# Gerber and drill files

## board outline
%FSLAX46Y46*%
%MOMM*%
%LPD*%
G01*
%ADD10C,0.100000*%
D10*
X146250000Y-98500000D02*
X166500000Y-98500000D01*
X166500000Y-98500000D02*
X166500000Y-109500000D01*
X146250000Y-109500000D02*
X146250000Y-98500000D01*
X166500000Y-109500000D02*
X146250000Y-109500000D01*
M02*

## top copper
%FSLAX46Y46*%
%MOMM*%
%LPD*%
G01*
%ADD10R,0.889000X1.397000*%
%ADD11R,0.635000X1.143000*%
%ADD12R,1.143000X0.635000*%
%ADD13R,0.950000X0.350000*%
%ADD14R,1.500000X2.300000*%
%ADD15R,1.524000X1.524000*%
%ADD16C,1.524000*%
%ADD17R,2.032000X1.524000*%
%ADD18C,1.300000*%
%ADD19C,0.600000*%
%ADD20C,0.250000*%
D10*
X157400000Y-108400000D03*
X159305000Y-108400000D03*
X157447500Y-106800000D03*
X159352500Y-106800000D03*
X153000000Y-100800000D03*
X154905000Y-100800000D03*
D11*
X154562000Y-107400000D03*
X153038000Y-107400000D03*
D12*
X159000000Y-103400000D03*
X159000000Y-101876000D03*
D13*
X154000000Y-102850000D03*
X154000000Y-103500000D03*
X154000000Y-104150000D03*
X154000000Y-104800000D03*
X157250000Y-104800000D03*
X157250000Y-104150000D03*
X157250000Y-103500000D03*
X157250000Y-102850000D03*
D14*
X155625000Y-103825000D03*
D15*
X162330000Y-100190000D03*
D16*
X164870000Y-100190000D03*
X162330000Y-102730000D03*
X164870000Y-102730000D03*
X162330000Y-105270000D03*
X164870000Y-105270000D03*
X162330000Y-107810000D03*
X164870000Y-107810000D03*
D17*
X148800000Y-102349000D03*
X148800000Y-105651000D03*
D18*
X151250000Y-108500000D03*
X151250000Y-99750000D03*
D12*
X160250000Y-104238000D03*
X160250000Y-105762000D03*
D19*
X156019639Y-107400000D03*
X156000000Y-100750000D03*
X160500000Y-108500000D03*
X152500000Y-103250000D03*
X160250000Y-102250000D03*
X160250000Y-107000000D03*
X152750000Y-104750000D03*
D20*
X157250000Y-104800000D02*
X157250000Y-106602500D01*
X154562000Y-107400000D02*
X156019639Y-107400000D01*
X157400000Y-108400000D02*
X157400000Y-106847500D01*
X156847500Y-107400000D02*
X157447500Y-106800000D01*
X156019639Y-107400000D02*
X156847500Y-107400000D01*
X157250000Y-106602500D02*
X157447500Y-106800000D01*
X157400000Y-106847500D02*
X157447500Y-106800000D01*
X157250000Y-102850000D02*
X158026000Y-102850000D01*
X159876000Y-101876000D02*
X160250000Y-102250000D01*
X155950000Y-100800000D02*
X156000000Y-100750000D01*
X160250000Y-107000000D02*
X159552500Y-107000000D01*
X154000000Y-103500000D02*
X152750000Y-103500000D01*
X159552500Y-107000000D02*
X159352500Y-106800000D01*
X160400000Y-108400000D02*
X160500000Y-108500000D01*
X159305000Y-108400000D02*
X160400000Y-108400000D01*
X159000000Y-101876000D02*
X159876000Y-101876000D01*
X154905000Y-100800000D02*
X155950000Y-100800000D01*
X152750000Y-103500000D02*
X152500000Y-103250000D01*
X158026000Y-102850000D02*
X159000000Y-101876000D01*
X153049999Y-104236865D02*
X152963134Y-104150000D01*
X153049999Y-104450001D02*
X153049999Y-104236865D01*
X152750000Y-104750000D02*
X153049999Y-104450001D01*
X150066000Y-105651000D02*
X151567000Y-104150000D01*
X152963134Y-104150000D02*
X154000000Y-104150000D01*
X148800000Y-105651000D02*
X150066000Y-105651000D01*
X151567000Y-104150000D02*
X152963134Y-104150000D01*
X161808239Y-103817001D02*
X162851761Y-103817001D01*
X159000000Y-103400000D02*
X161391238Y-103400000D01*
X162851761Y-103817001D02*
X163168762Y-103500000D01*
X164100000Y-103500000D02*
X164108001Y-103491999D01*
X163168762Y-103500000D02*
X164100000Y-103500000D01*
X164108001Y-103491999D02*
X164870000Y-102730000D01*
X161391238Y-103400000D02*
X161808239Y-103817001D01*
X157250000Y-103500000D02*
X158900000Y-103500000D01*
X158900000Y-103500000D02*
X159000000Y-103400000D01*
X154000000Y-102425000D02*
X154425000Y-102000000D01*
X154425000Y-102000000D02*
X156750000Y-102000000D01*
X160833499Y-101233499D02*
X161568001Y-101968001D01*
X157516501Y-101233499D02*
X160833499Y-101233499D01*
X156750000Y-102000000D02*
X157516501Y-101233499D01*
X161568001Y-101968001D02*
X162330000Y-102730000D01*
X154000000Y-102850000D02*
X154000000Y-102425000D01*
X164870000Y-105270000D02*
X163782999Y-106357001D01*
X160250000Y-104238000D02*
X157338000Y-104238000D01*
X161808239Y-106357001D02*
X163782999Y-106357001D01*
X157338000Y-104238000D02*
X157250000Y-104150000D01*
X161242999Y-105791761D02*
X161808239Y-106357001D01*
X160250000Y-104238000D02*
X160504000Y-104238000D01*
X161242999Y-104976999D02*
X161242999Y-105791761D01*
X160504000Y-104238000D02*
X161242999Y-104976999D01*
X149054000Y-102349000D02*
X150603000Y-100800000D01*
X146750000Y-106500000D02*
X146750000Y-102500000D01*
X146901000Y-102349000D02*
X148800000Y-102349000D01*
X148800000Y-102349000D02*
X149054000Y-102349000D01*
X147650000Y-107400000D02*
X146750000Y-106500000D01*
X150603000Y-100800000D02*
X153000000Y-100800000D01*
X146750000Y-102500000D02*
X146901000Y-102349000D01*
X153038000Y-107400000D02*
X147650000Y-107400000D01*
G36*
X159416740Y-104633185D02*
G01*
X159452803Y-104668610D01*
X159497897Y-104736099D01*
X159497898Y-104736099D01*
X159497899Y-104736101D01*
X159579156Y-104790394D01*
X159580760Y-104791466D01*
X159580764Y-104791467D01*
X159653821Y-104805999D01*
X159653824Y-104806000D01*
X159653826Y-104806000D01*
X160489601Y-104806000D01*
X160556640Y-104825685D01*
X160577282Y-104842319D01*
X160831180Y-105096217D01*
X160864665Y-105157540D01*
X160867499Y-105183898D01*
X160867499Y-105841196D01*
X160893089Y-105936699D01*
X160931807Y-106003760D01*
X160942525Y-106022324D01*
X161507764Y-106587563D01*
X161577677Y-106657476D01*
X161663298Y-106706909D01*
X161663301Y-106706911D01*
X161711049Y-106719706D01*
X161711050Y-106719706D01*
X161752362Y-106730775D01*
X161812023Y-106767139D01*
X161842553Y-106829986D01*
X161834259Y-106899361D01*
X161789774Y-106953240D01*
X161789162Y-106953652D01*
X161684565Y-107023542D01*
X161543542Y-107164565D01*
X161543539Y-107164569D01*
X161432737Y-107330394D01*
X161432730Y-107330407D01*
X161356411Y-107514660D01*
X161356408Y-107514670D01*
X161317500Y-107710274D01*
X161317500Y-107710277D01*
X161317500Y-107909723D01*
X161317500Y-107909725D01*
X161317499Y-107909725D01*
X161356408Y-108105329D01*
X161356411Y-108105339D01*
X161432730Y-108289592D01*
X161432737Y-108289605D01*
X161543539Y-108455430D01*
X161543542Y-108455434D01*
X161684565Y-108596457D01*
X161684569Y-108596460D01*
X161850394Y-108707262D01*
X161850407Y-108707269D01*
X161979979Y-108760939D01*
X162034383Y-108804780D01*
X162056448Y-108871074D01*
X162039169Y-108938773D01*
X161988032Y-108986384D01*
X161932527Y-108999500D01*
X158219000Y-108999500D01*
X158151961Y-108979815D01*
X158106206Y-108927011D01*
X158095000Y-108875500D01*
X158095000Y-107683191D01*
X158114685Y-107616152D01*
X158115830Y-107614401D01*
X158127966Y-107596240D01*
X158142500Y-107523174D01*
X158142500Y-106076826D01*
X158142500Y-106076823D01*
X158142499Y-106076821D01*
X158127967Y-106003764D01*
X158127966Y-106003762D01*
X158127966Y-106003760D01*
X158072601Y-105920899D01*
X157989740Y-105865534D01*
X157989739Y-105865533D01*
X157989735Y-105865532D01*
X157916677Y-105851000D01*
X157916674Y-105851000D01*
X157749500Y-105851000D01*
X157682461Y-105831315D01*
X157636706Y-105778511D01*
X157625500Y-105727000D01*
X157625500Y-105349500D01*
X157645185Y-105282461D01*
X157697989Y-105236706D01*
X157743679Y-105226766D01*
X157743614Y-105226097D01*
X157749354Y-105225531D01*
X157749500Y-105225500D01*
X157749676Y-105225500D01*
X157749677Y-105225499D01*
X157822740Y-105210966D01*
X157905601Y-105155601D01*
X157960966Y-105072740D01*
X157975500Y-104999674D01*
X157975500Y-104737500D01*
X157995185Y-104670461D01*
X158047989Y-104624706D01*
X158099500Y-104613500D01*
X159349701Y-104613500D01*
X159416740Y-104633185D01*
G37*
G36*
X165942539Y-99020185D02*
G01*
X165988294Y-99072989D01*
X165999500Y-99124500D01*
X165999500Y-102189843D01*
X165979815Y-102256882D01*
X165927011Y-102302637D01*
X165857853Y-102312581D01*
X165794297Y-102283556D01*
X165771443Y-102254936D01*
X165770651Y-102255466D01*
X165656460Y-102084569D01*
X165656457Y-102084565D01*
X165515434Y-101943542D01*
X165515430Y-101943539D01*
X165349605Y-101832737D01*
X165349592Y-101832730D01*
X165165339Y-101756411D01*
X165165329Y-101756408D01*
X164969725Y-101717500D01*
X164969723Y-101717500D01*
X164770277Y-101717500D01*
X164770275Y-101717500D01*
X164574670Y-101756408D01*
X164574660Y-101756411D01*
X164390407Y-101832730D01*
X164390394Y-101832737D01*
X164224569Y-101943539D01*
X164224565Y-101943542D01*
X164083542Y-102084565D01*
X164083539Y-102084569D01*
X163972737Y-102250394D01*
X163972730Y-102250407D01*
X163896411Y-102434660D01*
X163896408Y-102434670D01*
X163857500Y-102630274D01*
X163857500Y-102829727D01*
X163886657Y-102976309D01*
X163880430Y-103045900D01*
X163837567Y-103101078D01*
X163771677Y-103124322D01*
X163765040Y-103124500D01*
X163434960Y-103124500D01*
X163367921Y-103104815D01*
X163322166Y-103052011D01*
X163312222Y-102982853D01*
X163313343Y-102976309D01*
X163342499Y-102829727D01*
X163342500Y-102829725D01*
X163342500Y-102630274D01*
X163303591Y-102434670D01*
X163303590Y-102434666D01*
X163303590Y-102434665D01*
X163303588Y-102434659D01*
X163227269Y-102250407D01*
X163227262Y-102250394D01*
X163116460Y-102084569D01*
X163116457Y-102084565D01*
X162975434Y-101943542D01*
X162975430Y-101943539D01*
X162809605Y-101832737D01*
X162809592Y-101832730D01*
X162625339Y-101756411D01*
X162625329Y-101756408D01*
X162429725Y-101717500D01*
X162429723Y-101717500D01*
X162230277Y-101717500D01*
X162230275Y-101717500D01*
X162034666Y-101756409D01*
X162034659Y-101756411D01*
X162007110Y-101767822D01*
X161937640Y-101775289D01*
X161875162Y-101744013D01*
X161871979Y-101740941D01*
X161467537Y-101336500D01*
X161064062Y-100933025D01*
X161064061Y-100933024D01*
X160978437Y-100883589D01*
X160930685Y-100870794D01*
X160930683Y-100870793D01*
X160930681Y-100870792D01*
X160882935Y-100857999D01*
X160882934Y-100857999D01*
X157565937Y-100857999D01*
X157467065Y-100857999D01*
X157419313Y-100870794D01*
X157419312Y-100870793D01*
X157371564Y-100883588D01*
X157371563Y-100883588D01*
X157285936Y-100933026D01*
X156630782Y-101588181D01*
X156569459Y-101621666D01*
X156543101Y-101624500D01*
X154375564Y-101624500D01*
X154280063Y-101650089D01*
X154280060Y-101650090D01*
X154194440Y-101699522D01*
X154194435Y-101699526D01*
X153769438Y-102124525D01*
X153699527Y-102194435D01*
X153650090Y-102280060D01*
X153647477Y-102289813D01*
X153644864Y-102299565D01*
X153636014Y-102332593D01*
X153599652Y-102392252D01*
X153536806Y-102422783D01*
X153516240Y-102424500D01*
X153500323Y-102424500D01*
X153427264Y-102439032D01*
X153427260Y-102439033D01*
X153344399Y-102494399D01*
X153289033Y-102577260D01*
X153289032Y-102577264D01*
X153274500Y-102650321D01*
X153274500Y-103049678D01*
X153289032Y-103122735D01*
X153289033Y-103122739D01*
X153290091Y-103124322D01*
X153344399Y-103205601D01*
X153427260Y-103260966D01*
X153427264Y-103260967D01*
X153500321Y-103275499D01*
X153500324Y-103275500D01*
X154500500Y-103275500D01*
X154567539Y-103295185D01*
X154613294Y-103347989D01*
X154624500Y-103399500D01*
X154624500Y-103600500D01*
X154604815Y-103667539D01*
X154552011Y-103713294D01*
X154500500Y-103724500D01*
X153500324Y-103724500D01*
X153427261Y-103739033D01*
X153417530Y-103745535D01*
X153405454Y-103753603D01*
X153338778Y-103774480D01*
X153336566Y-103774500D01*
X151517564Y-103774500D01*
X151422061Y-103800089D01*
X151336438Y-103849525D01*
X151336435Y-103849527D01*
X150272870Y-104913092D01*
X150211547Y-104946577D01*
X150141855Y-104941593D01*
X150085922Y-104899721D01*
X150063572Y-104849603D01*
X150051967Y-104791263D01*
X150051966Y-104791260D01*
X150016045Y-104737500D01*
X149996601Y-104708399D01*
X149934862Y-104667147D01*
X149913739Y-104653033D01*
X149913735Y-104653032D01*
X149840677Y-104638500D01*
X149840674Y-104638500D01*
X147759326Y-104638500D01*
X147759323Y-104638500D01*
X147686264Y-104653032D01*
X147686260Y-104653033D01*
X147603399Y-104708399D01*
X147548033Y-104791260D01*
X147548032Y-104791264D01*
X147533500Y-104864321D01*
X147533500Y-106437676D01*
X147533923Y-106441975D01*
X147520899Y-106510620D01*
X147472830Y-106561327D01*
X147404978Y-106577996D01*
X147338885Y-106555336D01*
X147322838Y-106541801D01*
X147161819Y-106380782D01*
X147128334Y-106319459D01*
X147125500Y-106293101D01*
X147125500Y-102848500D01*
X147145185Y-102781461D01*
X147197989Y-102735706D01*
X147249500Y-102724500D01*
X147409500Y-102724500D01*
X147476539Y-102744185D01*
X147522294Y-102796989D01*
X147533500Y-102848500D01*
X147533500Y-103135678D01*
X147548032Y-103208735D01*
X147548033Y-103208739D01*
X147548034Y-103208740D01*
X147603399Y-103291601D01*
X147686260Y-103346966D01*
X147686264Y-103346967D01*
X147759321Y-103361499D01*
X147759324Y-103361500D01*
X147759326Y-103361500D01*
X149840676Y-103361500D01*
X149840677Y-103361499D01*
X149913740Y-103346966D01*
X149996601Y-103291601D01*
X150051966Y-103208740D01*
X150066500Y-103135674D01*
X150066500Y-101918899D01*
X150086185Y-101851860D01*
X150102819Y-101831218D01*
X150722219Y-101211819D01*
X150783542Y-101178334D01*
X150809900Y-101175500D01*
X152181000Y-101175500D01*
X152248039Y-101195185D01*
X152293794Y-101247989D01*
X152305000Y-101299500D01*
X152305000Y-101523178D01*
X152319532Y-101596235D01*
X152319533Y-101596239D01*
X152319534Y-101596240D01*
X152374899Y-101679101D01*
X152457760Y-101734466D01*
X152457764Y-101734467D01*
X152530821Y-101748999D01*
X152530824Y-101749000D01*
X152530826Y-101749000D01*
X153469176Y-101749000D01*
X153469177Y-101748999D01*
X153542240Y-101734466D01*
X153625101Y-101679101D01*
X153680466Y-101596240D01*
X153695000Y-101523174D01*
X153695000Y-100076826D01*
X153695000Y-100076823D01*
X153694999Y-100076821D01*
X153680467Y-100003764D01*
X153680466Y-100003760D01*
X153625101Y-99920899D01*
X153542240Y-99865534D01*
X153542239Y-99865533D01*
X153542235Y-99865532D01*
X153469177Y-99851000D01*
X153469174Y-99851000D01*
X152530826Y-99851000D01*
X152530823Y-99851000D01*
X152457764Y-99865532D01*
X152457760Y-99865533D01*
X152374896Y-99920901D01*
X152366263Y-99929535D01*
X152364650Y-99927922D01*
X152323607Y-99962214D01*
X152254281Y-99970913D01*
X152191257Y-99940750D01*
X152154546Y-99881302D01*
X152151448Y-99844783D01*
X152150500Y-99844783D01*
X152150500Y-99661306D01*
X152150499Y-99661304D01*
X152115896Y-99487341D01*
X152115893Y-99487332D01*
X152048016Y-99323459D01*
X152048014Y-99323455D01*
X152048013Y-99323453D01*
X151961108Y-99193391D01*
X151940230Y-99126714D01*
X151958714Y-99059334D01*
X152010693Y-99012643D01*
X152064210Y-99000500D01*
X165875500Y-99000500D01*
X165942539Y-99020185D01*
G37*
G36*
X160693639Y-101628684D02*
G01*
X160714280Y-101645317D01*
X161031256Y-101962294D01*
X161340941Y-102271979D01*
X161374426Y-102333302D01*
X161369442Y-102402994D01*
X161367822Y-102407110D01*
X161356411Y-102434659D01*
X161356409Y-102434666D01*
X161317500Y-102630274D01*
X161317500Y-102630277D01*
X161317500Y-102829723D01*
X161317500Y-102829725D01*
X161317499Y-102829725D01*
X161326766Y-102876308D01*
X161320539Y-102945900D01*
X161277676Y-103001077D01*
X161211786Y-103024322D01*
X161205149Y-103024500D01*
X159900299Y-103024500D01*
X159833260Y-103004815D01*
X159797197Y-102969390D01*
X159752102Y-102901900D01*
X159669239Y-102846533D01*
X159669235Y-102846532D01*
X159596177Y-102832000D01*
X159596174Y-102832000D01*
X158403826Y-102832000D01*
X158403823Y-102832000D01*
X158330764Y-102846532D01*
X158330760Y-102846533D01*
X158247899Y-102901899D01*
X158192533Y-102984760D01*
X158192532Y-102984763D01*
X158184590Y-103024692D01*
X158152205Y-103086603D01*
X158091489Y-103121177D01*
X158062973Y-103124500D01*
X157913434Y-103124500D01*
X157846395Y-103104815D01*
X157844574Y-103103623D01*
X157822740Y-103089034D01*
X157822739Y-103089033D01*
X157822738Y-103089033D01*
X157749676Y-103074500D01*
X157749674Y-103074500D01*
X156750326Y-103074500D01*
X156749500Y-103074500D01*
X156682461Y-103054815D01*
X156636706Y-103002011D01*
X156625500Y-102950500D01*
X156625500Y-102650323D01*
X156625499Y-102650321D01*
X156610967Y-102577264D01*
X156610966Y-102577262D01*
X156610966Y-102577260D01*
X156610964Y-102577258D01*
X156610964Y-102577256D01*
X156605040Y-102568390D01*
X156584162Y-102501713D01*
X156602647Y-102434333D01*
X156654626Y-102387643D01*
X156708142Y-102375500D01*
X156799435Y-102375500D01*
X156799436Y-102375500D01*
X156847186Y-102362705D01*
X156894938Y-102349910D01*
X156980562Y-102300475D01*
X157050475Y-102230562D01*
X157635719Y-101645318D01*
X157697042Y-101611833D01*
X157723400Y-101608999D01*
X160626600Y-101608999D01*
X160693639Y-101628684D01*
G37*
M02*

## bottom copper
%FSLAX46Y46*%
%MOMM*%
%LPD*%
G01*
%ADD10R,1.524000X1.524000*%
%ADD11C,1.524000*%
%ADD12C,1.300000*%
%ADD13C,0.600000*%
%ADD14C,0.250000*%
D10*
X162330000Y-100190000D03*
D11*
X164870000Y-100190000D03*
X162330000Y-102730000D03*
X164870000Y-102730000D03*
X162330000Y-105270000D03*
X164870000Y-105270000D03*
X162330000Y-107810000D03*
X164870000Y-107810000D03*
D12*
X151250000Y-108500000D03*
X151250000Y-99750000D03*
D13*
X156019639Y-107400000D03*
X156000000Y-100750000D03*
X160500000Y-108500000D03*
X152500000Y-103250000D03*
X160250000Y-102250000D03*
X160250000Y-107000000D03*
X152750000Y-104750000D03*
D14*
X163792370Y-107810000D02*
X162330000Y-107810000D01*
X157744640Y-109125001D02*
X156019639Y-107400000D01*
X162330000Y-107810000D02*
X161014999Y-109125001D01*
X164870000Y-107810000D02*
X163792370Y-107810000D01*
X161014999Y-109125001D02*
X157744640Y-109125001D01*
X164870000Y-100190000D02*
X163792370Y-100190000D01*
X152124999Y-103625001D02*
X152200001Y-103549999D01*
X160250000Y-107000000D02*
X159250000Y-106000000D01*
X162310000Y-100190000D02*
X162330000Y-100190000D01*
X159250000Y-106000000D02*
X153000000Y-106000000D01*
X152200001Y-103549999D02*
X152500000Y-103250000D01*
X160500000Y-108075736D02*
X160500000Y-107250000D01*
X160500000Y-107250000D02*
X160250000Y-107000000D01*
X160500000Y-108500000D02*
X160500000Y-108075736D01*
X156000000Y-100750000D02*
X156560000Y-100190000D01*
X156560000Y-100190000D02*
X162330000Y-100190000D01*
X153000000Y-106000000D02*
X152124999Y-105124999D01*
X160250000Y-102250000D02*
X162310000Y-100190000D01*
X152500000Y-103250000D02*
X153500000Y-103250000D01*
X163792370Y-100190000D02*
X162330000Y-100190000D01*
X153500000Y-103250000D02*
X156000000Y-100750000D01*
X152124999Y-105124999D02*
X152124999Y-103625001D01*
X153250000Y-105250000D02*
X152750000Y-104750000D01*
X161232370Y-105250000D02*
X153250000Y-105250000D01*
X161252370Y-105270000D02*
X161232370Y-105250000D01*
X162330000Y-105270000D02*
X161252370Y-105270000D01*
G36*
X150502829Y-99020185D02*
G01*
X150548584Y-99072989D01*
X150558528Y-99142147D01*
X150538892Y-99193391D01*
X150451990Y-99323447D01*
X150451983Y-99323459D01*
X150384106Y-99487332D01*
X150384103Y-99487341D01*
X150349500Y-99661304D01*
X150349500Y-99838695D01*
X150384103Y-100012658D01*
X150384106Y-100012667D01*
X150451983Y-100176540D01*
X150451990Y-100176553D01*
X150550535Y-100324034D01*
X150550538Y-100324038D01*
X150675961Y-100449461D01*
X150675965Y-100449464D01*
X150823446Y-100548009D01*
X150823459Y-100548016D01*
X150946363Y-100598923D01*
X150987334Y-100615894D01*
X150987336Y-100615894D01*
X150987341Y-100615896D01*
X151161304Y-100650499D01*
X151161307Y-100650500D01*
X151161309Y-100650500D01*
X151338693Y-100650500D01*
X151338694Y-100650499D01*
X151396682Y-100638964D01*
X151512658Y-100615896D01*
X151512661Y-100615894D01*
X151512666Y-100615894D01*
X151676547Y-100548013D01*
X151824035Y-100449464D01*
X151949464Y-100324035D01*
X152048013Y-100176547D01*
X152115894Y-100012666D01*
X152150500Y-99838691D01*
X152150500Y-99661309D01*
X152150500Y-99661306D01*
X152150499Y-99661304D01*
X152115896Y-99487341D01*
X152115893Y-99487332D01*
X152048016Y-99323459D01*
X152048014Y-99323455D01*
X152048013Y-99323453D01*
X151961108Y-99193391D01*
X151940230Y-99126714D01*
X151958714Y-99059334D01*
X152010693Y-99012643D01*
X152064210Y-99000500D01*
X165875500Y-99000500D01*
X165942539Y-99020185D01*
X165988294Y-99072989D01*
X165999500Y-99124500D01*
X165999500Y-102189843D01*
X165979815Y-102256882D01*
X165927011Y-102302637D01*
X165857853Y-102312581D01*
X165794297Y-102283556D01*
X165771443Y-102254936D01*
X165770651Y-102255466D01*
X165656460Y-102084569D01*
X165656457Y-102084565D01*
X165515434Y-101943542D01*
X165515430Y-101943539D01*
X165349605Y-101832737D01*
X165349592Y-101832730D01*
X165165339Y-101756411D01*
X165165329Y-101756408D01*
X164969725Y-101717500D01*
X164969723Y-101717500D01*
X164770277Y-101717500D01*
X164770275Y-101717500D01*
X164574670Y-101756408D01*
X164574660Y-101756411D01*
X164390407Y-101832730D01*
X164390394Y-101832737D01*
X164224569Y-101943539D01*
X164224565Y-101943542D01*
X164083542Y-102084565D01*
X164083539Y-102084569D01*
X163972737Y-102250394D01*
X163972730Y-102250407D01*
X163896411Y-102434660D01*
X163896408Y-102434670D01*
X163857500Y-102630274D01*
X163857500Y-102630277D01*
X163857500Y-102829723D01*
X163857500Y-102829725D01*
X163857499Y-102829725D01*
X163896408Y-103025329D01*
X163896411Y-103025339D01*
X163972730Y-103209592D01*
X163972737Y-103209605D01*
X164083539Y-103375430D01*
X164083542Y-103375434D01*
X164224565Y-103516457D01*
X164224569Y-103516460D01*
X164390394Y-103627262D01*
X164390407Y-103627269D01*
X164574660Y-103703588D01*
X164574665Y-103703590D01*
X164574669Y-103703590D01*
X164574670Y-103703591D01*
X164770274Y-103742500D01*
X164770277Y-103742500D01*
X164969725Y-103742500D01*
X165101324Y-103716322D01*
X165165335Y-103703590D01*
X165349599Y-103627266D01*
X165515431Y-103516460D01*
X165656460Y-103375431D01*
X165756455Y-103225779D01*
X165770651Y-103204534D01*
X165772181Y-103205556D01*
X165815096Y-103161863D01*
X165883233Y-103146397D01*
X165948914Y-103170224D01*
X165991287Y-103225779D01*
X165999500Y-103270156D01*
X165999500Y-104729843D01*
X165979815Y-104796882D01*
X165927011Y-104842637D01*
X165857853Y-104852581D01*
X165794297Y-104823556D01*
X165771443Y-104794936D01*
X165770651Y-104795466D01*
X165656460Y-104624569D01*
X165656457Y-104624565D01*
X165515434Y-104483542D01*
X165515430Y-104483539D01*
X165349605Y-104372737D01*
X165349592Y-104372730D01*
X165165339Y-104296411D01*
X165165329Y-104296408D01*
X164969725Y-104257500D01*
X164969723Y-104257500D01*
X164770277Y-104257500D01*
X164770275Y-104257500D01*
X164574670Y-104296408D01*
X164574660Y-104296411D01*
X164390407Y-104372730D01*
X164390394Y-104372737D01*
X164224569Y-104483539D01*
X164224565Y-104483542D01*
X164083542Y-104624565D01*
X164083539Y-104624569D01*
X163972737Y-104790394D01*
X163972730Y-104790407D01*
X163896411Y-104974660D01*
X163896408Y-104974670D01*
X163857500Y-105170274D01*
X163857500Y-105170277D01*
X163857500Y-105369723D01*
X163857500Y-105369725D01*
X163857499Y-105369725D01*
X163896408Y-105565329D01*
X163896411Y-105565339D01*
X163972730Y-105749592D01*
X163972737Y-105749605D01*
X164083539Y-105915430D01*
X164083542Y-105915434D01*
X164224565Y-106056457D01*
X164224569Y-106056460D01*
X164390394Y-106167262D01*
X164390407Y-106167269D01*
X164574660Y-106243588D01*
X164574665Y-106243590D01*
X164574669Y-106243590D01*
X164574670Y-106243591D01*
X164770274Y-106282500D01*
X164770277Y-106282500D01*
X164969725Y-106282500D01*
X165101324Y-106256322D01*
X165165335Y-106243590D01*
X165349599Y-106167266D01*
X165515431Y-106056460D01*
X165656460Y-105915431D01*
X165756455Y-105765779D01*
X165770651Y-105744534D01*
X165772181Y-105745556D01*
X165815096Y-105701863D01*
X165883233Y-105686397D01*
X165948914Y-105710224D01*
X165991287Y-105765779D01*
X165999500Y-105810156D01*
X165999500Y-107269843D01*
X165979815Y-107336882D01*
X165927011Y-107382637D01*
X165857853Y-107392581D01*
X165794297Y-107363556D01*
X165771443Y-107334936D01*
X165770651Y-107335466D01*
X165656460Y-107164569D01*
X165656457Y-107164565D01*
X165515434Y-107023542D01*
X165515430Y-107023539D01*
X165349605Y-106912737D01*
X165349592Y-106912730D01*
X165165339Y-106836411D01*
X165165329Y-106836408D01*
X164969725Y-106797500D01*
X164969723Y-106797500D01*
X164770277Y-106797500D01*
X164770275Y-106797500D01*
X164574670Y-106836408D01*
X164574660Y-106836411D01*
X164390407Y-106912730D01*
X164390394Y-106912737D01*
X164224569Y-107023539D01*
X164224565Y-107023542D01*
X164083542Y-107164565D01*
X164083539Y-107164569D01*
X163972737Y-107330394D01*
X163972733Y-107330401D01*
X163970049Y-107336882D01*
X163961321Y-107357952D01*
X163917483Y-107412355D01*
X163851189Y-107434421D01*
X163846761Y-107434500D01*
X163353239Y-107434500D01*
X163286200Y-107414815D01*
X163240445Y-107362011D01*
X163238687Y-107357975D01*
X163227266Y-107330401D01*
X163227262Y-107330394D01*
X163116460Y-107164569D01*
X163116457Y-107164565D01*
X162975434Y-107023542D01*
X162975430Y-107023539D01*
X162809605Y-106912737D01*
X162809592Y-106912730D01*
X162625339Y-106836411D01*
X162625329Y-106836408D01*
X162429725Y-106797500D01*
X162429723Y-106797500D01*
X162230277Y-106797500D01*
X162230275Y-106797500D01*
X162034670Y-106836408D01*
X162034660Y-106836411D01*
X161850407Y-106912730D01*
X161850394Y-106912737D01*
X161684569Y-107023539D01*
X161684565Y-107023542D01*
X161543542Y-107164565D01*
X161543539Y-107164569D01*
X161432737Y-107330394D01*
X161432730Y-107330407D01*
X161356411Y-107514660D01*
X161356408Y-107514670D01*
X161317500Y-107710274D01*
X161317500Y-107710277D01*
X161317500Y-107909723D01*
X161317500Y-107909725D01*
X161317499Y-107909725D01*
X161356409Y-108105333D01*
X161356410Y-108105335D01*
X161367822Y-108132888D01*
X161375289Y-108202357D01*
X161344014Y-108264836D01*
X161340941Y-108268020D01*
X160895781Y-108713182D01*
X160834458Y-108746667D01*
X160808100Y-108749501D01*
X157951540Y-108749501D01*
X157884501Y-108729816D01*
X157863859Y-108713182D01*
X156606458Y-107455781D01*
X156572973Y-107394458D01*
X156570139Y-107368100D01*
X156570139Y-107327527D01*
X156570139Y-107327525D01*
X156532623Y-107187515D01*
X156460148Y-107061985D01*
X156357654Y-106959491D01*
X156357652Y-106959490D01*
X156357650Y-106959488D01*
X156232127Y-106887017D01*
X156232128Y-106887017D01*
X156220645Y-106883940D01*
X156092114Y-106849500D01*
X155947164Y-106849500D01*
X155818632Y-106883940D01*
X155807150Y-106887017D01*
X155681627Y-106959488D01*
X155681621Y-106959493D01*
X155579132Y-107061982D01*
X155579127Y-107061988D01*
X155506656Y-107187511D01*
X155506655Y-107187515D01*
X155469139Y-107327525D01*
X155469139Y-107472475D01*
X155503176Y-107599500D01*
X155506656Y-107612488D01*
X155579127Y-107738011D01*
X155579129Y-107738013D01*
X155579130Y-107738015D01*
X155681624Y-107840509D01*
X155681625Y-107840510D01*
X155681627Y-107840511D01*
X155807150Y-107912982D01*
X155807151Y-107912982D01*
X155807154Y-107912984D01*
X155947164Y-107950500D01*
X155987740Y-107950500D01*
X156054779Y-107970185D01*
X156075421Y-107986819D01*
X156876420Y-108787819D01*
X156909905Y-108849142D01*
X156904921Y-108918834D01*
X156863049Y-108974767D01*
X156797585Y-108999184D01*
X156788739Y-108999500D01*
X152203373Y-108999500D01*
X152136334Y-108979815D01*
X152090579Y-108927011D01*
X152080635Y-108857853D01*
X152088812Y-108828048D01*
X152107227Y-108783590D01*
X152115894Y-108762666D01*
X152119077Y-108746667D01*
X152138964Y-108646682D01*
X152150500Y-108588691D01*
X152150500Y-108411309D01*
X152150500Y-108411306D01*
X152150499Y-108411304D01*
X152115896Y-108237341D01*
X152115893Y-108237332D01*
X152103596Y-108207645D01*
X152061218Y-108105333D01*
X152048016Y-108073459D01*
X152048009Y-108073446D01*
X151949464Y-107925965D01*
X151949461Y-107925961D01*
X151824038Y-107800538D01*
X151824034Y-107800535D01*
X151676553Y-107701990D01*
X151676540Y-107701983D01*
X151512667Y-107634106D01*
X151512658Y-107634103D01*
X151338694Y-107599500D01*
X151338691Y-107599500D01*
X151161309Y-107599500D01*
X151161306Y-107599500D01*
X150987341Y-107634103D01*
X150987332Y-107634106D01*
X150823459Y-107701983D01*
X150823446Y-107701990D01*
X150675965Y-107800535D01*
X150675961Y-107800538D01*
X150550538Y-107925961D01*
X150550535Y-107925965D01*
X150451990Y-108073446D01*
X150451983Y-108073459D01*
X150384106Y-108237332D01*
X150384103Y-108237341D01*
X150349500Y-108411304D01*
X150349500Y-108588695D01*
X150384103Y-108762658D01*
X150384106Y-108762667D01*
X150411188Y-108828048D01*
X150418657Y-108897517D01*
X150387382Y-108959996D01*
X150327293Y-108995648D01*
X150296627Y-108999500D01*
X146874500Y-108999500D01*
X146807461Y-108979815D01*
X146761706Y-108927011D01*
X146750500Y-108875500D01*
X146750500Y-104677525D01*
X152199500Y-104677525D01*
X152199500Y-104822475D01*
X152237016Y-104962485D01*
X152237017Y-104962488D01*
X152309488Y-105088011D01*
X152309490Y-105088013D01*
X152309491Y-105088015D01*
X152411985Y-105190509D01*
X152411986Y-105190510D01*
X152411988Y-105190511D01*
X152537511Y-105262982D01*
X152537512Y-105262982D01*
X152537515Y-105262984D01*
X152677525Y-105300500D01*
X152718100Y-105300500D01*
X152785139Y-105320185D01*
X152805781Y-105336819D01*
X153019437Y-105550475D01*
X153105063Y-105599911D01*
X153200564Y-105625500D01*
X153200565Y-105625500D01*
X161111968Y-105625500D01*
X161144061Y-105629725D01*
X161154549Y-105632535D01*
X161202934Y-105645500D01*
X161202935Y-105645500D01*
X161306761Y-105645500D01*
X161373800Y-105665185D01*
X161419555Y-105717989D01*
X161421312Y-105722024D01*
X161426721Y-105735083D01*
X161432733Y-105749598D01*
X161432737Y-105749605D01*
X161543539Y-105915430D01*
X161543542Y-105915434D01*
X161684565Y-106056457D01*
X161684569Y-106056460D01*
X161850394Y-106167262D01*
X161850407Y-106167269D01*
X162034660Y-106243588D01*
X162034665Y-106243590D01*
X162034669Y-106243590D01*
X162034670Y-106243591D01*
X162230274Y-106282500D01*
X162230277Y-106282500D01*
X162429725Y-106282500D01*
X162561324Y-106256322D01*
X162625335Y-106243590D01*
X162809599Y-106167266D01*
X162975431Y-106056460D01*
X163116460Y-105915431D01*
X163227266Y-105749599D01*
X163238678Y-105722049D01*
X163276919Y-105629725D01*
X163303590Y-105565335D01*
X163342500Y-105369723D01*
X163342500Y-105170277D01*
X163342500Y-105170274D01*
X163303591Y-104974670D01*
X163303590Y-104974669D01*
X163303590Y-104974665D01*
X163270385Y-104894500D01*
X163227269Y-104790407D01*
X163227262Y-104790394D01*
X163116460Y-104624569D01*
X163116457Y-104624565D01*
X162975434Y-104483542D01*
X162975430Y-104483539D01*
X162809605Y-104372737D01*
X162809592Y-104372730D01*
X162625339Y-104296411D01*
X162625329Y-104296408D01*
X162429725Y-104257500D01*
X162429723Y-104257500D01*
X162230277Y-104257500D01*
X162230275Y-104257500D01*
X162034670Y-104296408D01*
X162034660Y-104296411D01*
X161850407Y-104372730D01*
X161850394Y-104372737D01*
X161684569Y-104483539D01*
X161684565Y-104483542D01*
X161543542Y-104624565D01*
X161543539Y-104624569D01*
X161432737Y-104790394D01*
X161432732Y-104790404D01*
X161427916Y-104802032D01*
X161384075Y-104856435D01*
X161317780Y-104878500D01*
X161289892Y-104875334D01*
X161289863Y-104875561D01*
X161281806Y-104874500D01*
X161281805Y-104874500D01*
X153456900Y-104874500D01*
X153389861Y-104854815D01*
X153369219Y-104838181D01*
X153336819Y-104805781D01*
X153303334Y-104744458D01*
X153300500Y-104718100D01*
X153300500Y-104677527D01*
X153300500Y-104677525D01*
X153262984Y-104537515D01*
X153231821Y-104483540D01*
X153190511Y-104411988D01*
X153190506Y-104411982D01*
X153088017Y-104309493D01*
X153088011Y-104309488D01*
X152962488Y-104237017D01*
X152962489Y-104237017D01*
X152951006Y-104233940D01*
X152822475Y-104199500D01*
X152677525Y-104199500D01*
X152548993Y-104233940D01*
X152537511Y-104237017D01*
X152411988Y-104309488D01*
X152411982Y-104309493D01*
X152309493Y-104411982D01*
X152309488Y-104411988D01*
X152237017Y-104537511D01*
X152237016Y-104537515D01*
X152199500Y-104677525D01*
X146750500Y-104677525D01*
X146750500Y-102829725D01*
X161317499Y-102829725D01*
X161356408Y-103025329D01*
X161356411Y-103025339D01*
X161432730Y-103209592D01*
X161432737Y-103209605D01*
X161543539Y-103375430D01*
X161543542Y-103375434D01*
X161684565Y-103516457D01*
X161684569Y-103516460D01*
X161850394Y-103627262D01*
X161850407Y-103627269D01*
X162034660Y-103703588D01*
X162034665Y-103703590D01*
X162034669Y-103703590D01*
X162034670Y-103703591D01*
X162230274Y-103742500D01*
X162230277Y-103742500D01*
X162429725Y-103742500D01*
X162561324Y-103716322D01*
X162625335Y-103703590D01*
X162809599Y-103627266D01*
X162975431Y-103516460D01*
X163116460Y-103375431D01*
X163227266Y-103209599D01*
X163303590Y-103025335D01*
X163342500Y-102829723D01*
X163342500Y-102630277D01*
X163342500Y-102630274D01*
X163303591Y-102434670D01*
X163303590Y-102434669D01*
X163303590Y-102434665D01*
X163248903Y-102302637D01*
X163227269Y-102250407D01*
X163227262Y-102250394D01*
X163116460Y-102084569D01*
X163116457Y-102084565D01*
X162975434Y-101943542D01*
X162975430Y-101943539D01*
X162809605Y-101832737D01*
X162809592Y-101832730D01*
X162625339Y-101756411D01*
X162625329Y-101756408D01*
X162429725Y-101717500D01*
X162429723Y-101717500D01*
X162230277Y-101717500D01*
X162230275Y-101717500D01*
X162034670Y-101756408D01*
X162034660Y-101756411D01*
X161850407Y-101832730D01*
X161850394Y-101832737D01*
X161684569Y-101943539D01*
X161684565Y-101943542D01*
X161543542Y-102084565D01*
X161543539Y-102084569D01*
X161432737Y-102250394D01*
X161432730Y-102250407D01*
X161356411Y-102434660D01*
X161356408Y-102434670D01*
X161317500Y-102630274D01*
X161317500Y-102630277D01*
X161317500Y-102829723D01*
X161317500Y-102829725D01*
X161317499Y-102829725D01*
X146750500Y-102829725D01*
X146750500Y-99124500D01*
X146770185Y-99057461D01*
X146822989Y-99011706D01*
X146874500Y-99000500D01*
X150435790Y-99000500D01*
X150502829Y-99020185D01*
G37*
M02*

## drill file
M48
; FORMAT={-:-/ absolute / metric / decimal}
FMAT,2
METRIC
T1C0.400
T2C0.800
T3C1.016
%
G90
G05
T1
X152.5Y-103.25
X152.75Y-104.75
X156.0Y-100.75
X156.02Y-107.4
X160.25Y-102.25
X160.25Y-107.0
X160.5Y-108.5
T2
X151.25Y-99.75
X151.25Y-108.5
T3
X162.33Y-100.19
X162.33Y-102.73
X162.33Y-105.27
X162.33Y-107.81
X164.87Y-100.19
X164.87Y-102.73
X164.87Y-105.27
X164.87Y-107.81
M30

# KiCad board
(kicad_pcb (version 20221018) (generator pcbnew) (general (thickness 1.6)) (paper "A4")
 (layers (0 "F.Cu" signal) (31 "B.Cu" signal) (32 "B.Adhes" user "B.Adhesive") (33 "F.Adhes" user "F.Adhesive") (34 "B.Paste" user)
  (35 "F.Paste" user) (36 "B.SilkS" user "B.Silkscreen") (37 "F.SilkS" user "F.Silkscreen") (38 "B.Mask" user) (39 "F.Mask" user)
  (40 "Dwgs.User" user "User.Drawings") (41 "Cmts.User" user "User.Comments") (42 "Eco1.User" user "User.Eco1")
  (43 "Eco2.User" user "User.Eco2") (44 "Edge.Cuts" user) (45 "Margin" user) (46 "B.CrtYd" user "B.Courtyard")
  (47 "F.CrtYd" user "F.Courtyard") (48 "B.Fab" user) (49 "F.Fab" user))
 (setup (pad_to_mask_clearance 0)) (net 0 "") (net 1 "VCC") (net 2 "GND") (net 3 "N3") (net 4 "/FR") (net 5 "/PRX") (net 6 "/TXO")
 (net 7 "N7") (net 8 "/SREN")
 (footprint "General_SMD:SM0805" (layer "F.Cu") (at 158.3525 108.4)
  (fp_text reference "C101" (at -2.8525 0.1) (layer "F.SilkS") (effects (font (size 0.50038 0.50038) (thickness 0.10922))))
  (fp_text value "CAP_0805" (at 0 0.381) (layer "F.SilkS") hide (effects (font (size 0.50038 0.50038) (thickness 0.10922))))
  (pad "1" smd rect (at -0.9525 0) (size 0.889 1.397) (layers "F.Cu" "F.Paste" "F.Mask") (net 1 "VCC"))
  (pad "2" smd rect (at 0.9525 0) (size 0.889 1.397) (layers "F.Cu" "F.Paste" "F.Mask") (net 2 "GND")))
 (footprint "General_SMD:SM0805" (layer "F.Cu") (at 158.4 106.8)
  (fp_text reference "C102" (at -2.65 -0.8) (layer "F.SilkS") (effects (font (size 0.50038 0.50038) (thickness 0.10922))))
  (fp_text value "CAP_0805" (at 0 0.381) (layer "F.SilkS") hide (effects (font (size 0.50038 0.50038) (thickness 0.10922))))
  (pad "1" smd rect (at -0.9525 0) (size 0.889 1.397) (layers "F.Cu" "F.Paste" "F.Mask") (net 1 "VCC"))
  (pad "2" smd rect (at 0.9525 0) (size 0.889 1.397) (layers "F.Cu" "F.Paste" "F.Mask") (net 2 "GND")))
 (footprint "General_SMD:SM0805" (layer "F.Cu") (at 153.9525 100.8)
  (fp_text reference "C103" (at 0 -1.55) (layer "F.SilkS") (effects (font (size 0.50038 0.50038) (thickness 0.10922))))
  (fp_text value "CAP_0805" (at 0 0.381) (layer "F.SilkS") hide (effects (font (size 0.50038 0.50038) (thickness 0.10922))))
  (pad "1" smd rect (at -0.9525 0) (size 0.889 1.397) (layers "F.Cu" "F.Paste" "F.Mask") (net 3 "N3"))
  (pad "2" smd rect (at 0.9525 0) (size 0.889 1.397) (layers "F.Cu" "F.Paste" "F.Mask") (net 2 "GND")))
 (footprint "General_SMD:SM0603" (layer "F.Cu") (at 153.8 107.4 180)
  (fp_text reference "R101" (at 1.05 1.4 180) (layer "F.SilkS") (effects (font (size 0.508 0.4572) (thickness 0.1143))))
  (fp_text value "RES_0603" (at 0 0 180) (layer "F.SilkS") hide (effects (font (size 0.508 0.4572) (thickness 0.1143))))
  (pad "1" smd rect (at -0.762 0 180) (size 0.635 1.143) (layers "F.Cu" "F.Paste" "F.Mask") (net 1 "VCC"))
  (pad "2" smd rect (at 0.762 0 180) (size 0.635 1.143) (layers "F.Cu" "F.Paste" "F.Mask") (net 3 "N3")))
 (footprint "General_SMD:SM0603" (layer "F.Cu") (at 159 102.638 90)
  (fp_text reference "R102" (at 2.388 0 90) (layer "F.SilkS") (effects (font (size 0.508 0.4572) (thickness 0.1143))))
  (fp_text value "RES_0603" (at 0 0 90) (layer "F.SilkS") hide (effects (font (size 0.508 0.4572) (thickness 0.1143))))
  (pad "1" smd rect (at -0.762 0 90) (size 0.635 1.143) (layers "F.Cu" "F.Paste" "F.Mask") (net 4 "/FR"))
  (pad "2" smd rect (at 0.762 0 90) (size 0.635 1.143) (layers "F.Cu" "F.Paste" "F.Mask") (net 2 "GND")))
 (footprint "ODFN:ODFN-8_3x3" (layer "F.Cu") (at 155.625 103.825 -90)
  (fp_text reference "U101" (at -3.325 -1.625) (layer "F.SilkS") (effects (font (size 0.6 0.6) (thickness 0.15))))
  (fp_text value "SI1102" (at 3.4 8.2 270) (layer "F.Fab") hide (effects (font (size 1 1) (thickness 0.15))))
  (pad "1" smd rect (at -0.975 1.625 270) (size 0.35 0.95) (layers "F.Cu" "F.Paste" "F.Mask") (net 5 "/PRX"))
  (pad "2" smd rect (at -0.325 1.625 270) (size 0.35 0.95) (layers "F.Cu" "F.Paste" "F.Mask") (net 2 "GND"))
  (pad "3" smd rect (at 0.325 1.625 270) (size 0.35 0.95) (layers "F.Cu" "F.Paste" "F.Mask") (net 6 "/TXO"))
  (pad "4" smd rect (at 0.975 1.625 270) (size 0.35 0.95) (layers "F.Cu" "F.Paste" "F.Mask") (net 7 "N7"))
  (pad "5" smd rect (at 0.975 -1.625 270) (size 0.35 0.95) (layers "F.Cu" "F.Paste" "F.Mask") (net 1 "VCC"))
  (pad "6" smd rect (at 0.325 -1.625 270) (size 0.35 0.95) (layers "F.Cu" "F.Paste" "F.Mask") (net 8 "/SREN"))
  (pad "7" smd rect (at -0.325 -1.625 270) (size 0.35 0.95) (layers "F.Cu" "F.Paste" "F.Mask") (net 4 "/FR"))
  (pad "8" smd rect (at -0.975 -1.625 270) (size 0.35 0.95) (layers "F.Cu" "F.Paste" "F.Mask") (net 2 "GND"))
  (pad "9" smd rect (at 0 0 270) (size 2.3 1.5) (layers "F.Cu" "F.Paste" "F.Mask")))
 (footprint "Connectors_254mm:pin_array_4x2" (layer "F.Cu") (at 163.6 104 -90)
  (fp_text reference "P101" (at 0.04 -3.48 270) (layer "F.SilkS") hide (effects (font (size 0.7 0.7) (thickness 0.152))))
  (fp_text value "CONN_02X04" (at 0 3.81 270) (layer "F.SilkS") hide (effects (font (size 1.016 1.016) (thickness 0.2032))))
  (pad "1" thru_hole rect (at -3.81 1.27 270) (size 1.524 1.524) (drill 1.016) (layers "*.Cu" "*.Mask" "F.SilkS") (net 2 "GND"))
  (pad "2" thru_hole circle (at -3.81 -1.27 270) (size 1.524 1.524) (drill 1.016) (layers "*.Cu" "*.Mask" "F.SilkS") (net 2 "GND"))
  (pad "3" thru_hole circle (at -1.27 1.27 270) (size 1.524 1.524) (drill 1.016) (layers "*.Cu" "*.Mask" "F.SilkS") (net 5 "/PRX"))
  (pad "4" thru_hole circle (at -1.27 -1.27 270) (size 1.524 1.524) (drill 1.016) (layers "*.Cu" "*.Mask" "F.SilkS") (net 4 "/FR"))
  (pad "5" thru_hole circle (at 1.27 1.27 270) (size 1.524 1.524) (drill 1.016) (layers "*.Cu" "*.Mask" "F.SilkS") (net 6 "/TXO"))
  (pad "6" thru_hole circle (at 1.27 -1.27 270) (size 1.524 1.524) (drill 1.016) (layers "*.Cu" "*.Mask" "F.SilkS") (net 8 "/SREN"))
  (pad "7" thru_hole circle (at 3.81 1.27 270) (size 1.524 1.524) (drill 1.016) (layers "*.Cu" "*.Mask" "F.SilkS") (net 1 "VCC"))
  (pad "8" thru_hole circle (at 3.81 -1.27 270) (size 1.524 1.524) (drill 1.016) (layers "*.Cu" "*.Mask" "F.SilkS") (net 1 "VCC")))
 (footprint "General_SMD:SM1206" (layer "F.Cu") (at 148.8 104 -90)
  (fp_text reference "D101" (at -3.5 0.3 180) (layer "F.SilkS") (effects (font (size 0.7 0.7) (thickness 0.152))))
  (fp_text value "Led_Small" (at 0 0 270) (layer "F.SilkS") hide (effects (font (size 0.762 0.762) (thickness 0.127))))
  (pad "1" smd rect (at -1.651 0 270) (size 1.524 2.032) (layers "F.Cu" "F.Paste" "F.Mask") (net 3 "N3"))
  (pad "2" smd rect (at 1.651 0 270) (size 1.524 2.032) (layers "F.Cu" "F.Paste" "F.Mask") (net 6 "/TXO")))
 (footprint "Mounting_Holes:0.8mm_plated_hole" (layer "F.Cu") (at 151.25 108.5)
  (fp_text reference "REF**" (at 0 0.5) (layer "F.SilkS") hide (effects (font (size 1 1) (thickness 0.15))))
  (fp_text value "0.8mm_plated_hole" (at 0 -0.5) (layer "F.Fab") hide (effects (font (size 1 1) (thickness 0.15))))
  (pad "1" thru_hole circle (at 0 0) (size 1.3 1.3) (drill 0.8) (layers "*.Cu" "*.SilkS" "*.Mask")))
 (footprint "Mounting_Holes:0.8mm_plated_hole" (layer "F.Cu") (at 151.25 99.75)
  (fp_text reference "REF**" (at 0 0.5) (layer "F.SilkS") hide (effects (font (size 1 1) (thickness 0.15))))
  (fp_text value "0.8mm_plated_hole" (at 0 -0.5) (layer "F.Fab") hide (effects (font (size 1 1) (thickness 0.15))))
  (pad "1" thru_hole circle (at 0 0) (size 1.3 1.3) (drill 0.8) (layers "*.Cu" "*.SilkS" "*.Mask")))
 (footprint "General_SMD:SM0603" (layer "F.Cu") (at 160.25 105 -90)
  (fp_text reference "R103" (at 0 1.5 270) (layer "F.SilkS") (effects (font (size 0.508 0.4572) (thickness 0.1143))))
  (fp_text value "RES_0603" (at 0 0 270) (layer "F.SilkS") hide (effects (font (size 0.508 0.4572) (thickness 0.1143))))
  (pad "1" smd rect (at -0.762 0 270) (size 0.635 1.143) (layers "F.Cu" "F.Paste" "F.Mask") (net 8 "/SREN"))
  (pad "2" smd rect (at 0.762 0 270) (size 0.635 1.143) (layers "F.Cu" "F.Paste" "F.Mask") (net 2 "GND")))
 (gr_line (start 146.25 98.5) (end 166.5 98.5) (stroke (width 0.1) (type solid)) (layer "Edge.Cuts"))
 (gr_line (start 166.5 98.5) (end 166.5 109.5) (stroke (width 0.1) (type solid)) (layer "Edge.Cuts"))
 (gr_line (start 146.25 109.5) (end 146.25 98.5) (stroke (width 0.1) (type solid)) (layer "Edge.Cuts"))
 (gr_line (start 166.5 109.5) (end 146.25 109.5) (stroke (width 0.1) (type solid)) (layer "Edge.Cuts"))
 (segment (start 157.25 104.8) (end 157.25 106.6025) (width 0.25) (layer "F.Cu") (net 1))
 (segment (start 154.562 107.4) (end 156.019639 107.4) (width 0.25) (layer "F.Cu") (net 1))
 (segment (start 157.4 108.4) (end 157.4 106.8475) (width 0.25) (layer "F.Cu") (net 1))
 (segment (start 156.8475 107.4) (end 157.4475 106.8) (width 0.25) (layer "F.Cu") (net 1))
 (segment (start 156.019639 107.4) (end 156.8475 107.4) (width 0.25) (layer "F.Cu") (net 1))
 (segment (start 157.25 106.6025) (end 157.4475 106.8) (width 0.25) (layer "F.Cu") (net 1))
 (segment (start 157.4 106.8475) (end 157.4475 106.8) (width 0.25) (layer "F.Cu") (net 1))
 (via (at 156.019639 107.4) (size 0.6) (drill 0.4) (layers "F.Cu" "B.Cu") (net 1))
 (segment (start 163.79237 107.81) (end 162.33 107.81) (width 0.25) (layer "B.Cu") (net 1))
 (segment (start 157.74464 109.125001) (end 156.019639 107.4) (width 0.25) (layer "B.Cu") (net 1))
 (segment (start 162.33 107.81) (end 161.014999 109.125001) (width 0.25) (layer "B.Cu") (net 1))
 (segment (start 164.87 107.81) (end 163.79237 107.81) (width 0.25) (layer "B.Cu") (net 1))
 (segment (start 161.014999 109.125001) (end 157.74464 109.125001) (width 0.25) (layer "B.Cu") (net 1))
 (segment (start 157.25 102.85) (end 158.026 102.85) (width 0.25) (layer "F.Cu") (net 2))
 (segment (start 159.876 101.876) (end 160.25 102.25) (width 0.25) (layer "F.Cu") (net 2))
 (segment (start 155.95 100.8) (end 156 100.75) (width 0.25) (layer "F.Cu") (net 2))
 (segment (start 160.25 107) (end 159.5525 107) (width 0.25) (layer "F.Cu") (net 2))
 (segment (start 154 103.5) (end 152.75 103.5) (width 0.25) (layer "F.Cu") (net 2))
 (segment (start 159.5525 107) (end 159.3525 106.8) (width 0.25) (layer "F.Cu") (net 2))
 (segment (start 160.4 108.4) (end 160.5 108.5) (width 0.25) (layer "F.Cu") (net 2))
 (segment (start 159.305 108.4) (end 160.4 108.4) (width 0.25) (layer "F.Cu") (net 2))
 (segment (start 159 101.876) (end 159.876 101.876) (width 0.25) (layer "F.Cu") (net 2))
 (segment (start 154.905 100.8) (end 155.95 100.8) (width 0.25) (layer "F.Cu") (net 2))
 (segment (start 152.75 103.5) (end 152.5 103.25) (width 0.25) (layer "F.Cu") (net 2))
 (segment (start 158.026 102.85) (end 159 101.876) (width 0.25) (layer "F.Cu") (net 2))
 (via (at 156 100.75) (size 0.6) (drill 0.4) (layers "F.Cu" "B.Cu") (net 2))
 (via (at 160.5 108.5) (size 0.6) (drill 0.4) (layers "F.Cu" "B.Cu") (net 2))
 (via (at 152.5 103.25) (size 0.6) (drill 0.4) (layers "F.Cu" "B.Cu") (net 2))
 (via (at 160.25 102.25) (size 0.6) (drill 0.4) (layers "F.Cu" "B.Cu") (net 2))
 (via (at 160.25 107) (size 0.6) (drill 0.4) (layers "F.Cu" "B.Cu") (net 2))
 (segment (start 164.87 100.19) (end 163.79237 100.19) (width 0.25) (layer "B.Cu") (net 2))
 (segment (start 152.124999 103.625001) (end 152.200001 103.549999) (width 0.25) (layer "B.Cu") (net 2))
 (segment (start 160.25 107) (end 159.25 106) (width 0.25) (layer "B.Cu") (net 2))
 (segment (start 162.31 100.19) (end 162.33 100.19) (width 0.25) (layer "B.Cu") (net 2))
 (segment (start 159.25 106) (end 153 106) (width 0.25) (layer "B.Cu") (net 2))
 (segment (start 152.200001 103.549999) (end 152.5 103.25) (width 0.25) (layer "B.Cu") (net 2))
 (segment (start 160.5 108.075736) (end 160.5 107.25) (width 0.25) (layer "B.Cu") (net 2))
 (segment (start 160.5 107.25) (end 160.25 107) (width 0.25) (layer "B.Cu") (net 2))
 (segment (start 160.5 108.5) (end 160.5 108.075736) (width 0.25) (layer "B.Cu") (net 2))
 (segment (start 156 100.75) (end 156.56 100.19) (width 0.25) (layer "B.Cu") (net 2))
 (segment (start 156.56 100.19) (end 162.33 100.19) (width 0.25) (layer "B.Cu") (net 2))
 (segment (start 153 106) (end 152.124999 105.124999) (width 0.25) (layer "B.Cu") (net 2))
 (segment (start 160.25 102.25) (end 162.31 100.19) (width 0.25) (layer "B.Cu") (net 2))
 (segment (start 152.5 103.25) (end 153.5 103.25) (width 0.25) (layer "B.Cu") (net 2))
 (segment (start 163.79237 100.19) (end 162.33 100.19) (width 0.25) (layer "B.Cu") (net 2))
 (segment (start 153.5 103.25) (end 156 100.75) (width 0.25) (layer "B.Cu") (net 2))
 (segment (start 152.124999 105.124999) (end 152.124999 103.625001) (width 0.25) (layer "B.Cu") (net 2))
 (segment (start 153.049999 104.236865) (end 152.963134 104.15) (width 0.25) (layer "F.Cu") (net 6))
 (segment (start 153.049999 104.450001) (end 153.049999 104.236865) (width 0.25) (layer "F.Cu") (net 6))
 (segment (start 152.75 104.75) (end 153.049999 104.450001) (width 0.25) (layer "F.Cu") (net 6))
 (segment (start 150.066 105.651) (end 151.567 104.15) (width 0.25) (layer "F.Cu") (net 6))
 (segment (start 152.963134 104.15) (end 154 104.15) (width 0.25) (layer "F.Cu") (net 6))
 (segment (start 148.8 105.651) (end 150.066 105.651) (width 0.25) (layer "F.Cu") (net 6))
 (segment (start 151.567 104.15) (end 152.963134 104.15) (width 0.25) (layer "F.Cu") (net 6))
 (via (at 152.75 104.75) (size 0.6) (drill 0.4) (layers "F.Cu" "B.Cu") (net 6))
 (segment (start 153.25 105.25) (end 152.75 104.75) (width 0.25) (layer "B.Cu") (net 6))
 (segment (start 161.23237 105.25) (end 153.25 105.25) (width 0.25) (layer "B.Cu") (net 6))
 (segment (start 161.25237 105.27) (end 161.23237 105.25) (width 0.25) (layer "B.Cu") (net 6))
 (segment (start 162.33 105.27) (end 161.25237 105.27) (width 0.25) (layer "B.Cu") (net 6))
 (segment (start 161.808239 103.817001) (end 162.851761 103.817001) (width 0.25) (layer "F.Cu") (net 4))
 (segment (start 159 103.4) (end 161.391238 103.4) (width 0.25) (layer "F.Cu") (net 4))
 (segment (start 162.851761 103.817001) (end 163.168762 103.5) (width 0.25) (layer "F.Cu") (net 4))
 (segment (start 164.1 103.5) (end 164.108001 103.491999) (width 0.25) (layer "F.Cu") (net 4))
 (segment (start 163.168762 103.5) (end 164.1 103.5) (width 0.25) (layer "F.Cu") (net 4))
 (segment (start 164.108001 103.491999) (end 164.87 102.73) (width 0.25) (layer "F.Cu") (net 4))
 (segment (start 161.391238 103.4) (end 161.808239 103.817001) (width 0.25) (layer "F.Cu") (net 4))
 (segment (start 157.25 103.5) (end 158.9 103.5) (width 0.25) (layer "F.Cu") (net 4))
 (segment (start 158.9 103.5) (end 159 103.4) (width 0.25) (layer "F.Cu") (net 4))
 (segment (start 154 102.425) (end 154.425 102) (width 0.25) (layer "F.Cu") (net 5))
 (segment (start 154.425 102) (end 156.75 102) (width 0.25) (layer "F.Cu") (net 5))
 (segment (start 160.833499 101.233499) (end 161.568001 101.968001) (width 0.25) (layer "F.Cu") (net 5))
 (segment (start 157.516501 101.233499) (end 160.833499 101.233499) (width 0.25) (layer "F.Cu") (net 5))
 (segment (start 156.75 102) (end 157.516501 101.233499) (width 0.25) (layer "F.Cu") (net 5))
 (segment (start 161.568001 101.968001) (end 162.33 102.73) (width 0.25) (layer "F.Cu") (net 5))
 (segment (start 154 102.85) (end 154 102.425) (width 0.25) (layer "F.Cu") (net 5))
 (segment (start 164.87 105.27) (end 163.782999 106.357001) (width 0.25) (layer "F.Cu") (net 8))
 (segment (start 160.25 104.238) (end 157.338 104.238) (width 0.25) (layer "F.Cu") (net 8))
 (segment (start 161.808239 106.357001) (end 163.782999 106.357001) (width 0.25) (layer "F.Cu") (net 8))
 (segment (start 157.338 104.238) (end 157.25 104.15) (width 0.25) (layer "F.Cu") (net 8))
 (segment (start 161.242999 105.791761) (end 161.808239 106.357001) (width 0.25) (layer "F.Cu") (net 8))
 (segment (start 160.25 104.238) (end 160.504 104.238) (width 0.25) (layer "F.Cu") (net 8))
 (segment (start 161.242999 104.976999) (end 161.242999 105.791761) (width 0.25) (layer "F.Cu") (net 8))
 (segment (start 160.504 104.238) (end 161.242999 104.976999) (width 0.25) (layer "F.Cu") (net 8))
 (segment (start 149.054 102.349) (end 150.603 100.8) (width 0.25) (layer "F.Cu") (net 3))
 (segment (start 146.75 106.5) (end 146.75 102.5) (width 0.25) (layer "F.Cu") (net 3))
 (segment (start 146.901 102.349) (end 148.8 102.349) (width 0.25) (layer "F.Cu") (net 3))
 (segment (start 148.8 102.349) (end 149.054 102.349) (width 0.25) (layer "F.Cu") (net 3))
 (segment (start 147.65 107.4) (end 146.75 106.5) (width 0.25) (layer "F.Cu") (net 3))
 (segment (start 150.603 100.8) (end 153 100.8) (width 0.25) (layer "F.Cu") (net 3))
 (segment (start 146.75 102.5) (end 146.901 102.349) (width 0.25) (layer "F.Cu") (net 3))
 (segment (start 153.038 107.4) (end 147.65 107.4) (width 0.25) (layer "F.Cu") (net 3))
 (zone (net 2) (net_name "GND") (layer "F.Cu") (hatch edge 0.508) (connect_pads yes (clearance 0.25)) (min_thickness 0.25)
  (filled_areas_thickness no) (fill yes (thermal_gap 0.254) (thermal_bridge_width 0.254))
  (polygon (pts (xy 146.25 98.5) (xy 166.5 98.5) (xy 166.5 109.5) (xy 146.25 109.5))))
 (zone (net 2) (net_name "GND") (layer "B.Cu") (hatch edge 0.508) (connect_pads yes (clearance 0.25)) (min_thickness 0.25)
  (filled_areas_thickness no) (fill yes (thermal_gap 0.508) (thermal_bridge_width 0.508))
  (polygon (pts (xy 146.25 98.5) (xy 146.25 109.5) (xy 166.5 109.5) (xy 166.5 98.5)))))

